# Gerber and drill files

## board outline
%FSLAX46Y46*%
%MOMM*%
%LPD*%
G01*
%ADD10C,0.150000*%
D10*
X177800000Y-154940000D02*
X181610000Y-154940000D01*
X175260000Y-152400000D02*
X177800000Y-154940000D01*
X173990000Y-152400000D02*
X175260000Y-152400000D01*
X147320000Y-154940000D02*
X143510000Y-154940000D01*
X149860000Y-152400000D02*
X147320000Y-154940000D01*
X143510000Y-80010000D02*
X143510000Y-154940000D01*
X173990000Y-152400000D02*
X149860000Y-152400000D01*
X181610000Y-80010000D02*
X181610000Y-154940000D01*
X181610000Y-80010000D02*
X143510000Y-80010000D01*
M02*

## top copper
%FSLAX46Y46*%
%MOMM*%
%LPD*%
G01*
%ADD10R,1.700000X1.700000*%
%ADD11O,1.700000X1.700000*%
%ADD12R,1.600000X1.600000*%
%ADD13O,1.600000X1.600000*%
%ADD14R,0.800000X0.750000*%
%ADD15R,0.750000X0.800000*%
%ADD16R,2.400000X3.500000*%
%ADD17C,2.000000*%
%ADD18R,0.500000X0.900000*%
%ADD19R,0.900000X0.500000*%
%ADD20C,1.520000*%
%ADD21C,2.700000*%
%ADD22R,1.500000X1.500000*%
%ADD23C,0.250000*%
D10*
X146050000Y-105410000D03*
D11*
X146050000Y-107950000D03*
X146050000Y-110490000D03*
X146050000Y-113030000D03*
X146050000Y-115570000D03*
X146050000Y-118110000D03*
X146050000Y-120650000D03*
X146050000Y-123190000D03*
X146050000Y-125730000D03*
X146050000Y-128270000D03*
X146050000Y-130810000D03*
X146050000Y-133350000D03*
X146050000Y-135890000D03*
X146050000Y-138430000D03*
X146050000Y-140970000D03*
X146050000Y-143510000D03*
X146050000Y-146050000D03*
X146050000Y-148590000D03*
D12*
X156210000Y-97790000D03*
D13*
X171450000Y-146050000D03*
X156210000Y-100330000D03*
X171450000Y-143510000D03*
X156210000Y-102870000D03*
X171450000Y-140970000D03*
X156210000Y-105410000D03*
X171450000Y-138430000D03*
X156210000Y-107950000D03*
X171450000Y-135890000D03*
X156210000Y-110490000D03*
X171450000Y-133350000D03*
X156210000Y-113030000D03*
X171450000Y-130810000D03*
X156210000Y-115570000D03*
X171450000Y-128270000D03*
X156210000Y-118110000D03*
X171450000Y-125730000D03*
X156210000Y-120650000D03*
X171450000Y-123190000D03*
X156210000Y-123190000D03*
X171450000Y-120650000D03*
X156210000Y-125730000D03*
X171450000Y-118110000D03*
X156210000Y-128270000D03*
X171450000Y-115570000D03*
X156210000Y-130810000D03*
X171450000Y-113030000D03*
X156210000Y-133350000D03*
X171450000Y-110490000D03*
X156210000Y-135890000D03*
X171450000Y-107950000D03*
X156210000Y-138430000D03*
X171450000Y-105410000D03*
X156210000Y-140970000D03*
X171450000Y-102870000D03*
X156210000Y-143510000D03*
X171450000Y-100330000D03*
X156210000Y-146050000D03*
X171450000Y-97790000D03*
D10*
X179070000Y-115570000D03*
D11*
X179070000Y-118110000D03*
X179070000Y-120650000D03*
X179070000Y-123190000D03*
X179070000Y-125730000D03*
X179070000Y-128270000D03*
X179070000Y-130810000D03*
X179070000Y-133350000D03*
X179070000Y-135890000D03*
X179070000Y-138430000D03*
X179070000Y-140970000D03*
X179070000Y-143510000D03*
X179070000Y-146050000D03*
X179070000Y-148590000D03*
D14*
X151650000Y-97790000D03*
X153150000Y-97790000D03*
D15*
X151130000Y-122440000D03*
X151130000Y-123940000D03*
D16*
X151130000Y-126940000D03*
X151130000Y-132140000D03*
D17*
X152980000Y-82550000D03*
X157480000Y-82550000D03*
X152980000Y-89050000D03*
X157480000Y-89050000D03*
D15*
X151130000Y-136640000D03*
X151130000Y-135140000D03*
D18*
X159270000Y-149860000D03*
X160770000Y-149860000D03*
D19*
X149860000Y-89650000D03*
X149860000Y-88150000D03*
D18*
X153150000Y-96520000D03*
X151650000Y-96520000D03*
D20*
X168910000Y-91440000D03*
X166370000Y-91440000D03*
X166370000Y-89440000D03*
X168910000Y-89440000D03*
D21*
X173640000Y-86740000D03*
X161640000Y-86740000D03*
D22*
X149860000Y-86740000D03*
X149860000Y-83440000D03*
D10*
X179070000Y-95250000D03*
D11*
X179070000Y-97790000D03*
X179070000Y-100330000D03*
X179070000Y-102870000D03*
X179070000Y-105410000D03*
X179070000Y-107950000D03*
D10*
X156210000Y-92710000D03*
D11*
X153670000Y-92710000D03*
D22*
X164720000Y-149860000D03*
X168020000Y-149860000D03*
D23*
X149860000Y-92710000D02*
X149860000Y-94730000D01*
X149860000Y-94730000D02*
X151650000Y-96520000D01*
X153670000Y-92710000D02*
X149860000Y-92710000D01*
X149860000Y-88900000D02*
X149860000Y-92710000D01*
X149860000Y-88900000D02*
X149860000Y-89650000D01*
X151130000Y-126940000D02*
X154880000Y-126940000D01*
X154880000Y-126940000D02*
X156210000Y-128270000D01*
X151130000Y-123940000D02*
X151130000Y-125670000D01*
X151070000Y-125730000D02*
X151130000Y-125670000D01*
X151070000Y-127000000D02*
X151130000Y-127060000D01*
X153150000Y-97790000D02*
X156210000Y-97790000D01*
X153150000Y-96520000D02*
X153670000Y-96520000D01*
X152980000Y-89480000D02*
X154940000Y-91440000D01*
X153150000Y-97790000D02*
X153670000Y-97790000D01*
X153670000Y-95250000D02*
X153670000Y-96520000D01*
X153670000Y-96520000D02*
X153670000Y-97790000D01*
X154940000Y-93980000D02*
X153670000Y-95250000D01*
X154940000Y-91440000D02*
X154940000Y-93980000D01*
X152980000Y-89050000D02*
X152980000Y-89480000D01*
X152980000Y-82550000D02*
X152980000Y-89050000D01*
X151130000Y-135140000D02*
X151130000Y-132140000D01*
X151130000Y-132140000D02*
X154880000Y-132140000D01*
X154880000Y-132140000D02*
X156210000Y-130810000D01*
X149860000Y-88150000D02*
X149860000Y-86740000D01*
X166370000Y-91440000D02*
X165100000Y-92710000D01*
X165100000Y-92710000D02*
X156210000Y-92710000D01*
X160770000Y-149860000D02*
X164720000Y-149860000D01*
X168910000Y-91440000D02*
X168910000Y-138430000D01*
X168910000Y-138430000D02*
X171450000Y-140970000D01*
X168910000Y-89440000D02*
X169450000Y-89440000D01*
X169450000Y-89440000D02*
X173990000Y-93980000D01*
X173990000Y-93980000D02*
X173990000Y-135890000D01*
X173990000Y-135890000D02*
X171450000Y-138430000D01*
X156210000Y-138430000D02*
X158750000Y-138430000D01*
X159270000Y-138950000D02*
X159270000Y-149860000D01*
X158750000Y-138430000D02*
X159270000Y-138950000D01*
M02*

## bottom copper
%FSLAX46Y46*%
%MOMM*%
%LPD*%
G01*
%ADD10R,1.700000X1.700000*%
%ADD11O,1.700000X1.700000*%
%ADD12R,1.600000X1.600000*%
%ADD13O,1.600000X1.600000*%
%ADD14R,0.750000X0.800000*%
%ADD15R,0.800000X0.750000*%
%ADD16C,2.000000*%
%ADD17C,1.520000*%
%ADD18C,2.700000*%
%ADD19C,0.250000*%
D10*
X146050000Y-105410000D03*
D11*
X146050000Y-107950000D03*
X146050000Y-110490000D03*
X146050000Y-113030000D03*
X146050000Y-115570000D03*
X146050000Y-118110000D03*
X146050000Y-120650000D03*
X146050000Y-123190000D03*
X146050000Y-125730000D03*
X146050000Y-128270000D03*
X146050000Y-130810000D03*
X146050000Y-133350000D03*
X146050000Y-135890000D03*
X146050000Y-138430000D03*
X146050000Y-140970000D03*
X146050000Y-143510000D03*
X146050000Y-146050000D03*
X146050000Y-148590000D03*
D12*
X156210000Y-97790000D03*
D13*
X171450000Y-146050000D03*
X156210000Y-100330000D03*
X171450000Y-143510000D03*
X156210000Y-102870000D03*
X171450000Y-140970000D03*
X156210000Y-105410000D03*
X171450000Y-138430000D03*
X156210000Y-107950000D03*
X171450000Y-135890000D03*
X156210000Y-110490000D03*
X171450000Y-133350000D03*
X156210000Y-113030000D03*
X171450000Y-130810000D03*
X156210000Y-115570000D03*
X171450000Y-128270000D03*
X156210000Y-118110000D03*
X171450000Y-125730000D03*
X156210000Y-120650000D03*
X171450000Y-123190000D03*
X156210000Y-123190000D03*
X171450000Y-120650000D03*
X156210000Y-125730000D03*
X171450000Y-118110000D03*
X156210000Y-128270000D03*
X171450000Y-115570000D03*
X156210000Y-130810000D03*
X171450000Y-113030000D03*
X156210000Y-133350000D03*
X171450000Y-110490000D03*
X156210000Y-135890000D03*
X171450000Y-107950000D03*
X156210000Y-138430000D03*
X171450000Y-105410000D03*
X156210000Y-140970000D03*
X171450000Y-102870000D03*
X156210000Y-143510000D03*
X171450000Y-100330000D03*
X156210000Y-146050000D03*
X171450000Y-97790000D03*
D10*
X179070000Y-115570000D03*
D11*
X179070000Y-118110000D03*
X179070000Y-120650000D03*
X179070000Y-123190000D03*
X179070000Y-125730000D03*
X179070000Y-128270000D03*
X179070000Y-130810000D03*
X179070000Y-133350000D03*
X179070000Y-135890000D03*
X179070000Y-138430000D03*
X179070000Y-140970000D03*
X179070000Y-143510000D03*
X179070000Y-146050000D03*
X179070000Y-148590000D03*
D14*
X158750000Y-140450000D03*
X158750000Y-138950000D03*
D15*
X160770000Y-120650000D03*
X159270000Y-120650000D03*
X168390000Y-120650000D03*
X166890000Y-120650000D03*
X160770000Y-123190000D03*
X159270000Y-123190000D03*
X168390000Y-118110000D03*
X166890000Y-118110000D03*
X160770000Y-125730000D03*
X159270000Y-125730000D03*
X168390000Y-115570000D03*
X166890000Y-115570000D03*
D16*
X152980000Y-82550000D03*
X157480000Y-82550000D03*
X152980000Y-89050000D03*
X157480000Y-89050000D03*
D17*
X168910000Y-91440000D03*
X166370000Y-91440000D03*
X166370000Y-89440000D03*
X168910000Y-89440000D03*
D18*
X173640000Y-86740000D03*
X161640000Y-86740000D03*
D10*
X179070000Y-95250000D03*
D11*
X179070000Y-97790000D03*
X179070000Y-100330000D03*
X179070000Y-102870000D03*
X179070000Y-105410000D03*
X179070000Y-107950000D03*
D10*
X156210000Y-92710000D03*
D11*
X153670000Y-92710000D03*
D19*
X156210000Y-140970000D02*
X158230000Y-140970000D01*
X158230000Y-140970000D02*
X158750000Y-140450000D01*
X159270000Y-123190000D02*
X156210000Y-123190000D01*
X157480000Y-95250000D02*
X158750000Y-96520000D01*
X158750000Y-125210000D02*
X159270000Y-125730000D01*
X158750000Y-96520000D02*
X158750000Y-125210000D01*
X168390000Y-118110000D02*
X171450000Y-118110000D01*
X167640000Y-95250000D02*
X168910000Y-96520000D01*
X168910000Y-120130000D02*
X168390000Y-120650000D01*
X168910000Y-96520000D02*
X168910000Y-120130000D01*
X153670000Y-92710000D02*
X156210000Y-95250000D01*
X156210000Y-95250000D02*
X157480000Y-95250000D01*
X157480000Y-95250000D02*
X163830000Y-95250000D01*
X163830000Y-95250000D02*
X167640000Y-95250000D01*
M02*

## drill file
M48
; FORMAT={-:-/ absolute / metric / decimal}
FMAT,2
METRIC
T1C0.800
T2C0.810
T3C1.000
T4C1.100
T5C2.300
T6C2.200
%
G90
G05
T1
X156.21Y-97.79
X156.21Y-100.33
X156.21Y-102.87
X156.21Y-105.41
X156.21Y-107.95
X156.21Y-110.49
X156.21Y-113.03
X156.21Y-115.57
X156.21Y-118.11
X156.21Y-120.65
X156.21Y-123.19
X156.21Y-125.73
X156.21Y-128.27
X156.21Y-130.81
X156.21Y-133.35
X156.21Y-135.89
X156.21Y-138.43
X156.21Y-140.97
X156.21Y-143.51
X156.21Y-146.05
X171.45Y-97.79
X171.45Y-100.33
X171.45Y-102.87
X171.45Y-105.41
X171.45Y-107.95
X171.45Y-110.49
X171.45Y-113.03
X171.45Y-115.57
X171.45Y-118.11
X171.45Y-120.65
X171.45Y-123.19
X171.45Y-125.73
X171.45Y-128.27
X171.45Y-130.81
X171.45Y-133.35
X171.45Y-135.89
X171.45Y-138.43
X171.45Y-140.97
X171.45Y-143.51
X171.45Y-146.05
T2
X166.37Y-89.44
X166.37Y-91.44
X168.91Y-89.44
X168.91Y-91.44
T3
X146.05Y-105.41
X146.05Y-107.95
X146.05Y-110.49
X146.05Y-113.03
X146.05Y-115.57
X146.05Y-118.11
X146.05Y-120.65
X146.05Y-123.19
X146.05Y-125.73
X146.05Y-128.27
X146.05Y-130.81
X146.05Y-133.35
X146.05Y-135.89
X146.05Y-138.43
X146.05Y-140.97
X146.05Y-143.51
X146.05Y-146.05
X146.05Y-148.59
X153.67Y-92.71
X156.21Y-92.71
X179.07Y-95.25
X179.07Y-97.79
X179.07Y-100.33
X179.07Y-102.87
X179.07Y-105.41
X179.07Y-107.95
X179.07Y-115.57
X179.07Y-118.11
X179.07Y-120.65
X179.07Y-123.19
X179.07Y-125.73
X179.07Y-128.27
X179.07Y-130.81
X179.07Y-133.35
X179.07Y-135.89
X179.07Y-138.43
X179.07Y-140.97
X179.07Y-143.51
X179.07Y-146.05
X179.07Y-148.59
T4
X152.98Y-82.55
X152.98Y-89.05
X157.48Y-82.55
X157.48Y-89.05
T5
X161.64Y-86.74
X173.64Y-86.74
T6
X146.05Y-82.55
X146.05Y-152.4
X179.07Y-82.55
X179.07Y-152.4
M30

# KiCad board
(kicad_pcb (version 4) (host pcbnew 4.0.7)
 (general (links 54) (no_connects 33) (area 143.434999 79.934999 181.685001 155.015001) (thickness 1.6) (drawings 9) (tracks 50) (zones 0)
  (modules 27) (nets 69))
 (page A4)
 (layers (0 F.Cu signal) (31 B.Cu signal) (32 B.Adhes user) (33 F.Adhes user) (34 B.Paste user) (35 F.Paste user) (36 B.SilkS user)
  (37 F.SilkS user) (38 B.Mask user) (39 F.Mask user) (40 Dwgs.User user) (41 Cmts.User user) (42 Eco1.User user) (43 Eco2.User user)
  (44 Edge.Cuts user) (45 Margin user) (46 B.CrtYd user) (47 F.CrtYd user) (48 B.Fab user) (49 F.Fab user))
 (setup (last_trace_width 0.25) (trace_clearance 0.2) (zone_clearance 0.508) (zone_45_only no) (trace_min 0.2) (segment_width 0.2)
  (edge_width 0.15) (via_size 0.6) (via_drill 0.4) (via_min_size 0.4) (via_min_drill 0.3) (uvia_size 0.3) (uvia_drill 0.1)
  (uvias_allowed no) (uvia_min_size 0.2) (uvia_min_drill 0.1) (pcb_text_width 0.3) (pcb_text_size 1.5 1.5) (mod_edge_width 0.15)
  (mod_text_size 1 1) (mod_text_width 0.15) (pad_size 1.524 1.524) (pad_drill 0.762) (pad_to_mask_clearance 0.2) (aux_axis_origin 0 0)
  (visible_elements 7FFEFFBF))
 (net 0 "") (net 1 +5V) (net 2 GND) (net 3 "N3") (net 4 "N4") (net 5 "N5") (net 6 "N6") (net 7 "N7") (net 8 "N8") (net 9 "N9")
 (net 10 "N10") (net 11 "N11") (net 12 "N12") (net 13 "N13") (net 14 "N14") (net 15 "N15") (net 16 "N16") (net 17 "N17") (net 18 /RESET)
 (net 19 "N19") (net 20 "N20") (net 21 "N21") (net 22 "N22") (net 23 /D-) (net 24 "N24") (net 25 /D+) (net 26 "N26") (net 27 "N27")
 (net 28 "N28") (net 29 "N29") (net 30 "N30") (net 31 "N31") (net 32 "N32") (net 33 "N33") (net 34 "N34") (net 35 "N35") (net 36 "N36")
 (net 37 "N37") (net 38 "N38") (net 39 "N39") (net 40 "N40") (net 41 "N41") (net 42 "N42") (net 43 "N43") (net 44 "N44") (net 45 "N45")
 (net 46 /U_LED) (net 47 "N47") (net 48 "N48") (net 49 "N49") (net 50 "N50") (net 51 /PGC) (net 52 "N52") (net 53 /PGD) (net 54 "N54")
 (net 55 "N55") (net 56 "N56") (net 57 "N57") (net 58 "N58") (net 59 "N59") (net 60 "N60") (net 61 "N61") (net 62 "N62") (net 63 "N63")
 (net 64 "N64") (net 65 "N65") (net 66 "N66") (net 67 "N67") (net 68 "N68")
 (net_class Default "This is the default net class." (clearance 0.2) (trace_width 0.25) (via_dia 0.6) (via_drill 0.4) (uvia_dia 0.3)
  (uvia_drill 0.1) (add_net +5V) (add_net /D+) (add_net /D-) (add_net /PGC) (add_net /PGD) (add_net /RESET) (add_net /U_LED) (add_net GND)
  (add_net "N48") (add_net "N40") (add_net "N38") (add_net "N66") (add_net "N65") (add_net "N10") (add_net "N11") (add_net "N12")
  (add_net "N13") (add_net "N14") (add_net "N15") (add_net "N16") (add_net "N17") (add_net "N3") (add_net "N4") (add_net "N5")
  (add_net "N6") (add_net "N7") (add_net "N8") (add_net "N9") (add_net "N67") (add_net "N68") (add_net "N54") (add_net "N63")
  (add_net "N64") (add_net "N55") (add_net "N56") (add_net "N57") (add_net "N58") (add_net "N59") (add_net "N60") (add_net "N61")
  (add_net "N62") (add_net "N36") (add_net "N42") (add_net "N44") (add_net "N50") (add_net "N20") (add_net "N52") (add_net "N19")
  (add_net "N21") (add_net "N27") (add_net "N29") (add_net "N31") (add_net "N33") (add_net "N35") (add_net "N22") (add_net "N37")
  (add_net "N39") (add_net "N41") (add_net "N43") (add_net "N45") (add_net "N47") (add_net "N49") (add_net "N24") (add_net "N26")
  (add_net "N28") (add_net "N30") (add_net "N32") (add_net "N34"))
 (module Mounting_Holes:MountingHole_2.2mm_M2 (layer F.Cu) (at 146.05 82.55)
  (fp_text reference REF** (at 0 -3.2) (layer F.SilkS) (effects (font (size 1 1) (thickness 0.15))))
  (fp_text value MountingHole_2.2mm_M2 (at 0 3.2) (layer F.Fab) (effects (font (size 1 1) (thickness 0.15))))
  (pad 1 np_thru_hole circle (at 0 0) (size 2.2 2.2) (drill 2.2) (layers *.Cu *.Mask)))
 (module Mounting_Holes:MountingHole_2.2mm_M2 (layer F.Cu) (at 179.07 82.55)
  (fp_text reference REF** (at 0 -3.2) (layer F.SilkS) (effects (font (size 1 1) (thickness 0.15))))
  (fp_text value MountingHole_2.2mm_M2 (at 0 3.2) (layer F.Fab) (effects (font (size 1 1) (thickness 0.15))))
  (pad 1 np_thru_hole circle (at 0 0) (size 2.2 2.2) (drill 2.2) (layers *.Cu *.Mask)))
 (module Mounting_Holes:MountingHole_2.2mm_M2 (layer F.Cu) (at 179.07 152.4)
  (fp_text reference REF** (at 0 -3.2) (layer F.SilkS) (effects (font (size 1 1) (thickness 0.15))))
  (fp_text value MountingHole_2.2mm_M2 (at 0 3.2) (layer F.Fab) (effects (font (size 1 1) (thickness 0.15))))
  (pad 1 np_thru_hole circle (at 0 0) (size 2.2 2.2) (drill 2.2) (layers *.Cu *.Mask)))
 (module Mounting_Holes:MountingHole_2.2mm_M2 (layer F.Cu) (at 146.05 152.4)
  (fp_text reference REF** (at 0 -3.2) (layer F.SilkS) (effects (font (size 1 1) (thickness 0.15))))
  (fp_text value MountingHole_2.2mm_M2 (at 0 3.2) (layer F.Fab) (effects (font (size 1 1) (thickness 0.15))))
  (pad 1 np_thru_hole circle (at 0 0) (size 2.2 2.2) (drill 2.2) (layers *.Cu *.Mask)))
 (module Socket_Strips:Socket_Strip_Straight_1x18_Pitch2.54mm (layer F.Cu) (at 146.05 105.41)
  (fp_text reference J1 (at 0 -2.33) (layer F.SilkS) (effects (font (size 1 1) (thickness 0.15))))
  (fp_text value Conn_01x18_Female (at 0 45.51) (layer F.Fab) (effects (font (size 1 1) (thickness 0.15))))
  (pad 1 thru_hole rect (at 0 0) (size 1.7 1.7) (drill 1) (layers *.Cu *.Mask) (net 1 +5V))
  (pad 2 thru_hole oval (at 0 2.54) (size 1.7 1.7) (drill 1) (layers *.Cu *.Mask) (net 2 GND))
  (pad 3 thru_hole oval (at 0 5.08) (size 1.7 1.7) (drill 1) (layers *.Cu *.Mask) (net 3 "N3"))
  (pad 4 thru_hole oval (at 0 7.62) (size 1.7 1.7) (drill 1) (layers *.Cu *.Mask) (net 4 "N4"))
  (pad 5 thru_hole oval (at 0 10.16) (size 1.7 1.7) (drill 1) (layers *.Cu *.Mask) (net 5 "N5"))
  (pad 6 thru_hole oval (at 0 12.7) (size 1.7 1.7) (drill 1) (layers *.Cu *.Mask) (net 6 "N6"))
  (pad 7 thru_hole oval (at 0 15.24) (size 1.7 1.7) (drill 1) (layers *.Cu *.Mask) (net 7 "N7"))
  (pad 8 thru_hole oval (at 0 17.78) (size 1.7 1.7) (drill 1) (layers *.Cu *.Mask) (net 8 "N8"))
  (pad 9 thru_hole oval (at 0 20.32) (size 1.7 1.7) (drill 1) (layers *.Cu *.Mask) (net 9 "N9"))
  (pad 10 thru_hole oval (at 0 22.86) (size 1.7 1.7) (drill 1) (layers *.Cu *.Mask) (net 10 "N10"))
  (pad 11 thru_hole oval (at 0 25.4) (size 1.7 1.7) (drill 1) (layers *.Cu *.Mask) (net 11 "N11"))
  (pad 12 thru_hole oval (at 0 27.94) (size 1.7 1.7) (drill 1) (layers *.Cu *.Mask) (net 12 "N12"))
  (pad 13 thru_hole oval (at 0 30.48) (size 1.7 1.7) (drill 1) (layers *.Cu *.Mask) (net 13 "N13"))
  (pad 14 thru_hole oval (at 0 33.02) (size 1.7 1.7) (drill 1) (layers *.Cu *.Mask) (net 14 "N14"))
  (pad 15 thru_hole oval (at 0 35.56) (size 1.7 1.7) (drill 1) (layers *.Cu *.Mask) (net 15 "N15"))
  (pad 16 thru_hole oval (at 0 38.1) (size 1.7 1.7) (drill 1) (layers *.Cu *.Mask) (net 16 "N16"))
  (pad 17 thru_hole oval (at 0 40.64) (size 1.7 1.7) (drill 1) (layers *.Cu *.Mask) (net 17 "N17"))
  (pad 18 thru_hole oval (at 0 43.18) (size 1.7 1.7) (drill 1) (layers *.Cu *.Mask) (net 2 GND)))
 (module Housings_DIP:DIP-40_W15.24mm (layer F.Cu) (at 156.21 97.79)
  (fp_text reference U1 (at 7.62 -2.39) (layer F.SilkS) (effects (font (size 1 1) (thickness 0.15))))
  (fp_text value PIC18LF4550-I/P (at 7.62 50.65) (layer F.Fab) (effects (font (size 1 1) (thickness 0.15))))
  (pad 1 thru_hole rect (at 0 0) (size 1.6 1.6) (drill 0.8) (layers *.Cu *.Mask) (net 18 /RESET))
  (pad 21 thru_hole oval (at 15.24 48.26) (size 1.6 1.6) (drill 0.8) (layers *.Cu *.Mask) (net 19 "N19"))
  (pad 2 thru_hole oval (at 0 2.54) (size 1.6 1.6) (drill 0.8) (layers *.Cu *.Mask) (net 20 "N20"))
  (pad 22 thru_hole oval (at 15.24 45.72) (size 1.6 1.6) (drill 0.8) (layers *.Cu *.Mask) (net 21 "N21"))
  (pad 3 thru_hole oval (at 0 5.08) (size 1.6 1.6) (drill 0.8) (layers *.Cu *.Mask) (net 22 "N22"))
  (pad 23 thru_hole oval (at 15.24 43.18) (size 1.6 1.6) (drill 0.8) (layers *.Cu *.Mask) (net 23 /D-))
  (pad 4 thru_hole oval (at 0 7.62) (size 1.6 1.6) (drill 0.8) (layers *.Cu *.Mask) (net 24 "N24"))
  (pad 24 thru_hole oval (at 15.24 40.64) (size 1.6 1.6) (drill 0.8) (layers *.Cu *.Mask) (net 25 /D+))
  (pad 5 thru_hole oval (at 0 10.16) (size 1.6 1.6) (drill 0.8) (layers *.Cu *.Mask) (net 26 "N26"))
  (pad 25 thru_hole oval (at 15.24 38.1) (size 1.6 1.6) (drill 0.8) (layers *.Cu *.Mask) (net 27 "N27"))
  (pad 6 thru_hole oval (at 0 12.7) (size 1.6 1.6) (drill 0.8) (layers *.Cu *.Mask) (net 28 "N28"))
  (pad 26 thru_hole oval (at 15.24 35.56) (size 1.6 1.6) (drill 0.8) (layers *.Cu *.Mask) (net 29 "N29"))
  (pad 7 thru_hole oval (at 0 15.24) (size 1.6 1.6) (drill 0.8) (layers *.Cu *.Mask) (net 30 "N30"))
  (pad 27 thru_hole oval (at 15.24 33.02) (size 1.6 1.6) (drill 0.8) (layers *.Cu *.Mask) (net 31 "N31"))
  (pad 8 thru_hole oval (at 0 17.78) (size 1.6 1.6) (drill 0.8) (layers *.Cu *.Mask) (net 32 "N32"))
  (pad 28 thru_hole oval (at 15.24 30.48) (size 1.6 1.6) (drill 0.8) (layers *.Cu *.Mask) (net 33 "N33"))
  (pad 9 thru_hole oval (at 0 20.32) (size 1.6 1.6) (drill 0.8) (layers *.Cu *.Mask) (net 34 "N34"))
  (pad 29 thru_hole oval (at 15.24 27.94) (size 1.6 1.6) (drill 0.8) (layers *.Cu *.Mask) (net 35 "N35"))
  (pad 10 thru_hole oval (at 0 22.86) (size 1.6 1.6) (drill 0.8) (layers *.Cu *.Mask) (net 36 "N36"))
  (pad 30 thru_hole oval (at 15.24 25.4) (size 1.6 1.6) (drill 0.8) (layers *.Cu *.Mask) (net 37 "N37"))
  (pad 11 thru_hole oval (at 0 25.4) (size 1.6 1.6) (drill 0.8) (layers *.Cu *.Mask) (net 1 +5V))
  (pad 31 thru_hole oval (at 15.24 22.86) (size 1.6 1.6) (drill 0.8) (layers *.Cu *.Mask) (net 2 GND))
  (pad 12 thru_hole oval (at 0 27.94) (size 1.6 1.6) (drill 0.8) (layers *.Cu *.Mask) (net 2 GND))
  (pad 32 thru_hole oval (at 15.24 20.32) (size 1.6 1.6) (drill 0.8) (layers *.Cu *.Mask) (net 1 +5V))
  (pad 13 thru_hole oval (at 0 30.48) (size 1.6 1.6) (drill 0.8) (layers *.Cu *.Mask) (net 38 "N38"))
  (pad 33 thru_hole oval (at 15.24 17.78) (size 1.6 1.6) (drill 0.8) (layers *.Cu *.Mask) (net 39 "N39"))
  (pad 14 thru_hole oval (at 0 33.02) (size 1.6 1.6) (drill 0.8) (layers *.Cu *.Mask) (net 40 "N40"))
  (pad 34 thru_hole oval (at 15.24 15.24) (size 1.6 1.6) (drill 0.8) (layers *.Cu *.Mask) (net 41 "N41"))
  (pad 15 thru_hole oval (at 0 35.56) (size 1.6 1.6) (drill 0.8) (layers *.Cu *.Mask) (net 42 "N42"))
  (pad 35 thru_hole oval (at 15.24 12.7) (size 1.6 1.6) (drill 0.8) (layers *.Cu *.Mask) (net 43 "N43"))
  (pad 16 thru_hole oval (at 0 38.1) (size 1.6 1.6) (drill 0.8) (layers *.Cu *.Mask) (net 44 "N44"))
  (pad 36 thru_hole oval (at 15.24 10.16) (size 1.6 1.6) (drill 0.8) (layers *.Cu *.Mask) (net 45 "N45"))
  (pad 17 thru_hole oval (at 0 40.64) (size 1.6 1.6) (drill 0.8) (layers *.Cu *.Mask) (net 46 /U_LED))
  (pad 37 thru_hole oval (at 15.24 7.62) (size 1.6 1.6) (drill 0.8) (layers *.Cu *.Mask) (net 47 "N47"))
  (pad 18 thru_hole oval (at 0 43.18) (size 1.6 1.6) (drill 0.8) (layers *.Cu *.Mask) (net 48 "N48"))
  (pad 38 thru_hole oval (at 15.24 5.08) (size 1.6 1.6) (drill 0.8) (layers *.Cu *.Mask) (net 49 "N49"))
  (pad 19 thru_hole oval (at 0 45.72) (size 1.6 1.6) (drill 0.8) (layers *.Cu *.Mask) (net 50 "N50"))
  (pad 39 thru_hole oval (at 15.24 2.54) (size 1.6 1.6) (drill 0.8) (layers *.Cu *.Mask) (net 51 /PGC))
  (pad 20 thru_hole oval (at 0 48.26) (size 1.6 1.6) (drill 0.8) (layers *.Cu *.Mask) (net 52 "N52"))
  (pad 40 thru_hole oval (at 15.24 0) (size 1.6 1.6) (drill 0.8) (layers *.Cu *.Mask) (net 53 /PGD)))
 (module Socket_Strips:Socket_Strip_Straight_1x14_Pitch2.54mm (layer F.Cu) (at 179.07 115.57)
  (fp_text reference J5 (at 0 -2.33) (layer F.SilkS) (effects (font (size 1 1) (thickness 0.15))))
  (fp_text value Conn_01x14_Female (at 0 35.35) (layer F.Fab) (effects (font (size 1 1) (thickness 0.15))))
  (pad 1 thru_hole rect (at 0 0) (size 1.7 1.7) (drill 1) (layers *.Cu *.Mask) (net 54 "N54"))
  (pad 2 thru_hole oval (at 0 2.54) (size 1.7 1.7) (drill 1) (layers *.Cu *.Mask) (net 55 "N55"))
  (pad 3 thru_hole oval (at 0 5.08) (size 1.7 1.7) (drill 1) (layers *.Cu *.Mask) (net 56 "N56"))
  (pad 4 thru_hole oval (at 0 7.62) (size 1.7 1.7) (drill 1) (layers *.Cu *.Mask) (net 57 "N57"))
  (pad 5 thru_hole oval (at 0 10.16) (size 1.7 1.7) (drill 1) (layers *.Cu *.Mask) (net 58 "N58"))
  (pad 6 thru_hole oval (at 0 12.7) (size 1.7 1.7) (drill 1) (layers *.Cu *.Mask) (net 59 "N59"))
  (pad 7 thru_hole oval (at 0 15.24) (size 1.7 1.7) (drill 1) (layers *.Cu *.Mask) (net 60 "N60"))
  (pad 8 thru_hole oval (at 0 17.78) (size 1.7 1.7) (drill 1) (layers *.Cu *.Mask) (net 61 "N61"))
  (pad 9 thru_hole oval (at 0 20.32) (size 1.7 1.7) (drill 1) (layers *.Cu *.Mask) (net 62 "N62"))
  (pad 10 thru_hole oval (at 0 22.86) (size 1.7 1.7) (drill 1) (layers *.Cu *.Mask) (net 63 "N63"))
  (pad 11 thru_hole oval (at 0 25.4) (size 1.7 1.7) (drill 1) (layers *.Cu *.Mask) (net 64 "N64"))
  (pad 12 thru_hole oval (at 0 27.94) (size 1.7 1.7) (drill 1) (layers *.Cu *.Mask) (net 25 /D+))
  (pad 13 thru_hole oval (at 0 30.48) (size 1.7 1.7) (drill 1) (layers *.Cu *.Mask) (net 23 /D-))
  (pad 14 thru_hole oval (at 0 33.02) (size 1.7 1.7) (drill 1) (layers *.Cu *.Mask) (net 2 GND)))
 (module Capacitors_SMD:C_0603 (layer B.Cu) (at 158.75 139.7 270)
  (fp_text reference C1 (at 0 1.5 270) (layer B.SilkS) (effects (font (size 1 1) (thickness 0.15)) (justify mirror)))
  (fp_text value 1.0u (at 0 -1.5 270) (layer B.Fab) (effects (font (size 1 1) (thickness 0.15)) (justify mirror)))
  (pad 2 smd rect (at 0.75 0 270) (size 0.8 0.75) (layers B.Cu B.Paste B.Mask) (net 48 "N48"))
  (pad 1 smd rect (at -0.75 0 270) (size 0.8 0.75) (layers B.Cu B.Paste B.Mask) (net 2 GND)))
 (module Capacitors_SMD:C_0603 (layer F.Cu) (at 152.4 97.79 180)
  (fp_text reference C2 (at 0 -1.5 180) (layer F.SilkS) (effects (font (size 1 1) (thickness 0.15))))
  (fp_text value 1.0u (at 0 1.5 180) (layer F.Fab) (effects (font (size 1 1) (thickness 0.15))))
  (pad 2 smd rect (at 0.75 0 180) (size 0.8 0.75) (layers F.Cu F.Paste F.Mask) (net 2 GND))
  (pad 1 smd rect (at -0.75 0 180) (size 0.8 0.75) (layers F.Cu F.Paste F.Mask) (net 18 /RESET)))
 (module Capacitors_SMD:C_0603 (layer B.Cu) (at 160.02 120.65)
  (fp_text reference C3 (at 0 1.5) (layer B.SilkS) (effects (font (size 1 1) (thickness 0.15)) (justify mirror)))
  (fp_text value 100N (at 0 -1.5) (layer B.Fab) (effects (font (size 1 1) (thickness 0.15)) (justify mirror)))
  (pad 2 smd rect (at 0.75 0) (size 0.8 0.75) (layers B.Cu B.Paste B.Mask) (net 2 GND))
  (pad 1 smd rect (at -0.75 0) (size 0.8 0.75) (layers B.Cu B.Paste B.Mask) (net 1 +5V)))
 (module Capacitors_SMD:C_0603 (layer B.Cu) (at 167.64 120.65)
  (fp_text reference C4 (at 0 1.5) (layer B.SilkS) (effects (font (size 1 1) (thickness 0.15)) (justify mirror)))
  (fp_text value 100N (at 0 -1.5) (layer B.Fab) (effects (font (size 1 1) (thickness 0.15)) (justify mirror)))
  (pad 2 smd rect (at 0.75 0) (size 0.8 0.75) (layers B.Cu B.Paste B.Mask) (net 1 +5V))
  (pad 1 smd rect (at -0.75 0) (size 0.8 0.75) (layers B.Cu B.Paste B.Mask) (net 2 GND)))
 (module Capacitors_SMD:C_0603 (layer B.Cu) (at 160.02 123.19)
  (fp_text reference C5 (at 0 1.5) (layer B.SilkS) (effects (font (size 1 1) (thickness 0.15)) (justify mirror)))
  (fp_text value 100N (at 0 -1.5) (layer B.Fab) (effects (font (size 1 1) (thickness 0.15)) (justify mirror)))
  (pad 2 smd rect (at 0.75 0) (size 0.8 0.75) (layers B.Cu B.Paste B.Mask) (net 2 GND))
  (pad 1 smd rect (at -0.75 0) (size 0.8 0.75) (layers B.Cu B.Paste B.Mask) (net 1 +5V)))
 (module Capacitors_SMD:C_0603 (layer B.Cu) (at 167.64 118.11)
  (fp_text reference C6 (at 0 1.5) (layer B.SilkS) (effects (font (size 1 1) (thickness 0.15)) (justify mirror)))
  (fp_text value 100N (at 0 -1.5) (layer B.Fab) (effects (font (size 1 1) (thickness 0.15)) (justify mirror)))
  (pad 2 smd rect (at 0.75 0) (size 0.8 0.75) (layers B.Cu B.Paste B.Mask) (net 1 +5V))
  (pad 1 smd rect (at -0.75 0) (size 0.8 0.75) (layers B.Cu B.Paste B.Mask) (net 2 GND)))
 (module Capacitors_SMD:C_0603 (layer B.Cu) (at 160.02 125.73)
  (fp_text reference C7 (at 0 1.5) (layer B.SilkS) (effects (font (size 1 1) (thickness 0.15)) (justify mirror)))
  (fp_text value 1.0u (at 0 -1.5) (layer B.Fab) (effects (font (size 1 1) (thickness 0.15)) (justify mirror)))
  (pad 2 smd rect (at 0.75 0) (size 0.8 0.75) (layers B.Cu B.Paste B.Mask) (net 2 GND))
  (pad 1 smd rect (at -0.75 0) (size 0.8 0.75) (layers B.Cu B.Paste B.Mask) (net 1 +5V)))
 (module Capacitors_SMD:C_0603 (layer B.Cu) (at 167.64 115.57)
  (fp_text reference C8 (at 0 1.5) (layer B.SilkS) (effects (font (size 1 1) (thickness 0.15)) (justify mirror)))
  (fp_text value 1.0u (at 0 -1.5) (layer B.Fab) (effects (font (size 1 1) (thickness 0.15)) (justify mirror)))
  (pad 2 smd rect (at 0.75 0) (size 0.8 0.75) (layers B.Cu B.Paste B.Mask) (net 1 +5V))
  (pad 1 smd rect (at -0.75 0) (size 0.8 0.75) (layers B.Cu B.Paste B.Mask) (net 2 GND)))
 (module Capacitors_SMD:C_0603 (layer F.Cu) (at 151.13 123.19 90)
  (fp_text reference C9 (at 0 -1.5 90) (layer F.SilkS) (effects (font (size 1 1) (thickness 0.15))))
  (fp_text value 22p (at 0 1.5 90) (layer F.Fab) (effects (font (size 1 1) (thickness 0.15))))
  (pad 2 smd rect (at 0.75 0 90) (size 0.8 0.75) (layers F.Cu F.Paste F.Mask) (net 2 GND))
  (pad 1 smd rect (at -0.75 0 90) (size 0.8 0.75) (layers F.Cu F.Paste F.Mask) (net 38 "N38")))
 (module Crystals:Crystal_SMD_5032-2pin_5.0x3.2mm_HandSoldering (layer F.Cu) (at 151.13 129.54 270)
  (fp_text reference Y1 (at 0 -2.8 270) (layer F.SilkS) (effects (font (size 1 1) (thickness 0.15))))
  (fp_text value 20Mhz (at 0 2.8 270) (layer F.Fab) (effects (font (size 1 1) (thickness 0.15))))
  (pad 1 smd rect (at -2.6 0 270) (size 3.5 2.4) (layers F.Cu F.Paste F.Mask) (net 38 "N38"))
  (pad 2 smd rect (at 2.6 0 270) (size 3.5 2.4) (layers F.Cu F.Paste F.Mask) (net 40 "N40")))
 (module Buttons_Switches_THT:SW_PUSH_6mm (layer F.Cu) (at 157.48 82.55 270)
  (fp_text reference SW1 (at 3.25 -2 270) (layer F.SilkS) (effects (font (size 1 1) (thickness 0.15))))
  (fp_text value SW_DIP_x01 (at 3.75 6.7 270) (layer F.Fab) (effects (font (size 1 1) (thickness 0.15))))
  (pad 2 thru_hole circle (at 0 4.5) (size 2 2) (drill 1.1) (layers *.Cu *.Mask) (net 18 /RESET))
  (pad 1 thru_hole circle (at 0 0) (size 2 2) (drill 1.1) (layers *.Cu *.Mask) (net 2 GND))
  (pad 2 thru_hole circle (at 6.5 4.5) (size 2 2) (drill 1.1) (layers *.Cu *.Mask) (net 18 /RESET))
  (pad 1 thru_hole circle (at 6.5 0) (size 2 2) (drill 1.1) (layers *.Cu *.Mask) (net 2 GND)))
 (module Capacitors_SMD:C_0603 (layer F.Cu) (at 151.13 135.89 270)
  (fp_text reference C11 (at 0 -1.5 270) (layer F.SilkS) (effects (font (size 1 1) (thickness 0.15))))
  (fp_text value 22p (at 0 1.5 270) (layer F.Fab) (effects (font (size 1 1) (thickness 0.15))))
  (pad 2 smd rect (at 0.75 0 270) (size 0.8 0.75) (layers F.Cu F.Paste F.Mask) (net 2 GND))
  (pad 1 smd rect (at -0.75 0 270) (size 0.8 0.75) (layers F.Cu F.Paste F.Mask) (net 40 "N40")))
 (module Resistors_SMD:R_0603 (layer F.Cu) (at 160.02 149.86)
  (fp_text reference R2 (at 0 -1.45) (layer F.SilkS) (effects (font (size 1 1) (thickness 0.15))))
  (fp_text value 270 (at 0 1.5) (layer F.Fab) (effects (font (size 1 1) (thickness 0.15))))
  (pad 1 smd rect (at -0.75 0) (size 0.5 0.9) (layers F.Cu F.Paste F.Mask) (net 46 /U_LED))
  (pad 2 smd rect (at 0.75 0) (size 0.5 0.9) (layers F.Cu F.Paste F.Mask) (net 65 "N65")))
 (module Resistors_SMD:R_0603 (layer F.Cu) (at 149.86 88.9 90)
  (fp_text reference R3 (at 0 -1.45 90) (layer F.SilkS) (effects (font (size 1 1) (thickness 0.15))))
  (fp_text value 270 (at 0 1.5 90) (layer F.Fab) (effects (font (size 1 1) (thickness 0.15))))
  (pad 1 smd rect (at -0.75 0 90) (size 0.5 0.9) (layers F.Cu F.Paste F.Mask) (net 1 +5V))
  (pad 2 smd rect (at 0.75 0 90) (size 0.5 0.9) (layers F.Cu F.Paste F.Mask) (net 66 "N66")))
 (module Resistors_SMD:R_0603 (layer F.Cu) (at 152.4 96.52 180)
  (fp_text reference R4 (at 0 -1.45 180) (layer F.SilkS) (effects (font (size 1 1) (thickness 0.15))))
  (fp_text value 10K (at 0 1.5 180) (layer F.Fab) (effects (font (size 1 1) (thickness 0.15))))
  (pad 1 smd rect (at -0.75 0 180) (size 0.5 0.9) (layers F.Cu F.Paste F.Mask) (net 18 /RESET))
  (pad 2 smd rect (at 0.75 0 180) (size 0.5 0.9) (layers F.Cu F.Paste F.Mask) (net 1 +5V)))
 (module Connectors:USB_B (layer F.Cu) (at 166.37 91.44 90)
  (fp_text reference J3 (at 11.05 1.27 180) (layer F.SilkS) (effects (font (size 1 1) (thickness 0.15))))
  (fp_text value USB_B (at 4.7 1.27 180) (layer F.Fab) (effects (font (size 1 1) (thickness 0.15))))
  (pad 2 thru_hole circle (at 0 2.54) (size 1.52 1.52) (drill 0.81) (layers *.Cu *.Mask) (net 23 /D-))
  (pad 1 thru_hole circle (at 0 0) (size 1.52 1.52) (drill 0.81) (layers *.Cu *.Mask) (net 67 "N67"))
  (pad 4 thru_hole circle (at 2 0) (size 1.52 1.52) (drill 0.81) (layers *.Cu *.Mask) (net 2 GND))
  (pad 3 thru_hole circle (at 2 2.54) (size 1.52 1.52) (drill 0.81) (layers *.Cu *.Mask) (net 25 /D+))
  (pad 5 thru_hole circle (at 4.7 7.27) (size 2.7 2.7) (drill 2.3) (layers *.Cu *.Mask) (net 2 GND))
  (pad 5 thru_hole circle (at 4.7 -4.73) (size 2.7 2.7) (drill 2.3) (layers *.Cu *.Mask) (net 2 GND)))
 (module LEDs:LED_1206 (layer F.Cu) (at 149.86 85.09 270)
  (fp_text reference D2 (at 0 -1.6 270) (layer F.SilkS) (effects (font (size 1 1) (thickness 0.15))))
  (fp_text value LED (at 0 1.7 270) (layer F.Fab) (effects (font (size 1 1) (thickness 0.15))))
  (pad 2 smd rect (at 1.65 0 90) (size 1.5 1.5) (layers F.Cu F.Paste F.Mask) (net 66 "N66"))
  (pad 1 smd rect (at -1.65 0 90) (size 1.5 1.5) (layers F.Cu F.Paste F.Mask) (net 2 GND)))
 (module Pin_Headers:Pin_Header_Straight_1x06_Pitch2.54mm (layer F.Cu) (at 179.07 95.25)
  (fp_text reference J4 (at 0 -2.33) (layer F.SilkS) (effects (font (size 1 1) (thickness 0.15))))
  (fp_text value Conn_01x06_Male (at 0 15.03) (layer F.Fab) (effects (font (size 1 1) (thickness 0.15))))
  (pad 1 thru_hole rect (at 0 0) (size 1.7 1.7) (drill 1) (layers *.Cu *.Mask) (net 18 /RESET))
  (pad 2 thru_hole oval (at 0 2.54) (size 1.7 1.7) (drill 1) (layers *.Cu *.Mask) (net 1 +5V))
  (pad 3 thru_hole oval (at 0 5.08) (size 1.7 1.7) (drill 1) (layers *.Cu *.Mask) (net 2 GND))
  (pad 4 thru_hole oval (at 0 7.62) (size 1.7 1.7) (drill 1) (layers *.Cu *.Mask) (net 53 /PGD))
  (pad 5 thru_hole oval (at 0 10.16) (size 1.7 1.7) (drill 1) (layers *.Cu *.Mask) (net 51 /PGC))
  (pad 6 thru_hole oval (at 0 12.7) (size 1.7 1.7) (drill 1) (layers *.Cu *.Mask) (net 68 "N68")))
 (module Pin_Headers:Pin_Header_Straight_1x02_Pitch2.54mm (layer F.Cu) (at 156.21 92.71 270)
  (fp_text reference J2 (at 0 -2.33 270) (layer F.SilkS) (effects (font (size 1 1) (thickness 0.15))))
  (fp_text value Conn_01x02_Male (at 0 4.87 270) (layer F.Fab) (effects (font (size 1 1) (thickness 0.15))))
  (pad 1 thru_hole rect (at 0 0 270) (size 1.7 1.7) (drill 1) (layers *.Cu *.Mask) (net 67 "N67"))
  (pad 2 thru_hole oval (at 0 2.54 270) (size 1.7 1.7) (drill 1) (layers *.Cu *.Mask) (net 1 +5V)))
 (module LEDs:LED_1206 (layer F.Cu) (at 166.37 149.86 180)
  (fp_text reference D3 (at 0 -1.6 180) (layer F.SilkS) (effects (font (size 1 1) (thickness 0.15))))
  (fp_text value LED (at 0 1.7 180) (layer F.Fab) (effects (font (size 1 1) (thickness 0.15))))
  (pad 2 smd rect (at 1.65 0) (size 1.5 1.5) (layers F.Cu F.Paste F.Mask) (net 65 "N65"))
  (pad 1 smd rect (at -1.65 0) (size 1.5 1.5) (layers F.Cu F.Paste F.Mask) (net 2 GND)))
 (gr_line (start 177.8 154.94) (end 181.61 154.94) (angle 90) (layer Edge.Cuts) (width 0.15))
 (gr_line (start 175.26 152.4) (end 177.8 154.94) (angle 90) (layer Edge.Cuts) (width 0.15))
 (gr_line (start 173.99 152.4) (end 175.26 152.4) (angle 90) (layer Edge.Cuts) (width 0.15))
 (gr_line (start 147.32 154.94) (end 143.51 154.94) (angle 90) (layer Edge.Cuts) (width 0.15))
 (gr_line (start 149.86 152.4) (end 147.32 154.94) (angle 90) (layer Edge.Cuts) (width 0.15))
 (gr_line (start 143.51 80.01) (end 143.51 154.94) (angle 90) (layer Edge.Cuts) (width 0.15))
 (gr_line (start 173.99 152.4) (end 149.86 152.4) (angle 90) (layer Edge.Cuts) (width 0.15))
 (gr_line (start 181.61 80.01) (end 181.61 154.94) (angle 90) (layer Edge.Cuts) (width 0.15))
 (gr_line (start 181.61 80.01) (end 143.51 80.01) (angle 90) (layer Edge.Cuts) (width 0.15))
 (segment (start 156.21 140.97) (end 158.23 140.97) (width 0.25) (layer B.Cu) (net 48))
 (segment (start 158.23 140.97) (end 158.75 140.45) (width 0.25) (layer B.Cu) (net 48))
 (segment (start 159.27 123.19) (end 156.21 123.19) (width 0.25) (layer B.Cu) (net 1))
 (segment (start 157.48 95.25) (end 158.75 96.52) (width 0.25) (layer B.Cu) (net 1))
 (segment (start 158.75 125.21) (end 159.27 125.73) (width 0.25) (layer B.Cu) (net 1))
 (segment (start 158.75 96.52) (end 158.75 125.21) (width 0.25) (layer B.Cu) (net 1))
 (segment (start 168.39 118.11) (end 171.45 118.11) (width 0.25) (layer B.Cu) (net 1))
 (segment (start 167.64 95.25) (end 168.91 96.52) (width 0.25) (layer B.Cu) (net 1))
 (segment (start 168.91 120.13) (end 168.39 120.65) (width 0.25) (layer B.Cu) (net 1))
 (segment (start 168.91 96.52) (end 168.91 120.13) (width 0.25) (layer B.Cu) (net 1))
 (segment (start 149.86 92.71) (end 149.86 94.73) (width 0.25) (layer F.Cu) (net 1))
 (segment (start 149.86 94.73) (end 151.65 96.52) (width 0.25) (layer F.Cu) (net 1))
 (segment (start 153.67 92.71) (end 156.21 95.25) (width 0.25) (layer B.Cu) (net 1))
 (segment (start 156.21 95.25) (end 157.48 95.25) (width 0.25) (layer B.Cu) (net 1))
 (segment (start 157.48 95.25) (end 163.83 95.25) (width 0.25) (layer B.Cu) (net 1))
 (segment (start 163.83 95.25) (end 167.64 95.25) (width 0.25) (layer B.Cu) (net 1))
 (segment (start 153.67 92.71) (end 149.86 92.71) (width 0.25) (layer F.Cu) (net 1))
 (segment (start 149.86 88.9) (end 149.86 92.71) (width 0.25) (layer F.Cu) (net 1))
 (segment (start 149.86 88.9) (end 149.86 89.65) (width 0.25) (layer F.Cu) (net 1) (status 20))
 (segment (start 151.13 126.94) (end 154.88 126.94) (width 0.25) (layer F.Cu) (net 38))
 (segment (start 154.88 126.94) (end 156.21 128.27) (width 0.25) (layer F.Cu) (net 38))
 (segment (start 151.13 123.94) (end 151.13 125.67) (width 0.25) (layer F.Cu) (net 38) (status 10))
 (segment (start 151.07 125.73) (end 151.13 125.67) (width 0.25) (layer F.Cu) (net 38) (status 30))
 (segment (start 151.07 127) (end 151.13 127.06) (width 0.25) (layer F.Cu) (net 38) (status 30))
 (segment (start 153.15 97.79) (end 156.21 97.79) (width 0.25) (layer F.Cu) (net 18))
 (segment (start 153.15 96.52) (end 153.67 96.52) (width 0.25) (layer F.Cu) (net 18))
 (segment (start 152.98 89.48) (end 154.94 91.44) (width 0.25) (layer F.Cu) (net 18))
 (segment (start 153.15 97.79) (end 153.67 97.79) (width 0.25) (layer F.Cu) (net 18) (status 10))
 (segment (start 153.67 95.25) (end 153.67 96.52) (width 0.25) (layer F.Cu) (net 18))
 (segment (start 153.67 96.52) (end 153.67 97.79) (width 0.25) (layer F.Cu) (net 18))
 (segment (start 154.94 93.98) (end 153.67 95.25) (width 0.25) (layer F.Cu) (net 18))
 (segment (start 154.94 91.44) (end 154.94 93.98) (width 0.25) (layer F.Cu) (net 18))
 (segment (start 152.98 89.05) (end 152.98 89.48) (width 0.25) (layer F.Cu) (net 18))
 (segment (start 152.98 82.55) (end 152.98 89.05) (width 0.25) (layer F.Cu) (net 18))
 (segment (start 151.13 135.14) (end 151.13 132.14) (width 0.25) (layer F.Cu) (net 40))
 (segment (start 151.13 132.14) (end 154.88 132.14) (width 0.25) (layer F.Cu) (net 40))
 (segment (start 154.88 132.14) (end 156.21 130.81) (width 0.25) (layer F.Cu) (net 40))
 (segment (start 149.86 88.15) (end 149.86 86.74) (width 0.25) (layer F.Cu) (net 66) (status 20))
 (segment (start 166.37 91.44) (end 165.1 92.71) (width 0.25) (layer F.Cu) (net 67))
 (segment (start 165.1 92.71) (end 156.21 92.71) (width 0.25) (layer F.Cu) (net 67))
 (segment (start 160.77 149.86) (end 164.72 149.86) (width 0.25) (layer F.Cu) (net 65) (status C00000))
 (segment (start 168.91 91.44) (end 168.91 138.43) (width 0.25) (layer F.Cu) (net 23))
 (segment (start 168.91 138.43) (end 171.45 140.97) (width 0.25) (layer F.Cu) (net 23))
 (segment (start 168.91 89.44) (end 169.45 89.44) (width 0.25) (layer F.Cu) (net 25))
 (segment (start 169.45 89.44) (end 173.99 93.98) (width 0.25) (layer F.Cu) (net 25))
 (segment (start 173.99 93.98) (end 173.99 135.89) (width 0.25) (layer F.Cu) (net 25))
 (segment (start 173.99 135.89) (end 171.45 138.43) (width 0.25) (layer F.Cu) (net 25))
 (segment (start 156.21 138.43) (end 158.75 138.43) (width 0.25) (layer F.Cu) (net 46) (status 400000))
 (segment (start 159.27 138.95) (end 159.27 149.86) (width 0.25) (layer F.Cu) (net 46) (status 800000))
 (segment (start 158.75 138.43) (end 159.27 138.95) (width 0.25) (layer F.Cu) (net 46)))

